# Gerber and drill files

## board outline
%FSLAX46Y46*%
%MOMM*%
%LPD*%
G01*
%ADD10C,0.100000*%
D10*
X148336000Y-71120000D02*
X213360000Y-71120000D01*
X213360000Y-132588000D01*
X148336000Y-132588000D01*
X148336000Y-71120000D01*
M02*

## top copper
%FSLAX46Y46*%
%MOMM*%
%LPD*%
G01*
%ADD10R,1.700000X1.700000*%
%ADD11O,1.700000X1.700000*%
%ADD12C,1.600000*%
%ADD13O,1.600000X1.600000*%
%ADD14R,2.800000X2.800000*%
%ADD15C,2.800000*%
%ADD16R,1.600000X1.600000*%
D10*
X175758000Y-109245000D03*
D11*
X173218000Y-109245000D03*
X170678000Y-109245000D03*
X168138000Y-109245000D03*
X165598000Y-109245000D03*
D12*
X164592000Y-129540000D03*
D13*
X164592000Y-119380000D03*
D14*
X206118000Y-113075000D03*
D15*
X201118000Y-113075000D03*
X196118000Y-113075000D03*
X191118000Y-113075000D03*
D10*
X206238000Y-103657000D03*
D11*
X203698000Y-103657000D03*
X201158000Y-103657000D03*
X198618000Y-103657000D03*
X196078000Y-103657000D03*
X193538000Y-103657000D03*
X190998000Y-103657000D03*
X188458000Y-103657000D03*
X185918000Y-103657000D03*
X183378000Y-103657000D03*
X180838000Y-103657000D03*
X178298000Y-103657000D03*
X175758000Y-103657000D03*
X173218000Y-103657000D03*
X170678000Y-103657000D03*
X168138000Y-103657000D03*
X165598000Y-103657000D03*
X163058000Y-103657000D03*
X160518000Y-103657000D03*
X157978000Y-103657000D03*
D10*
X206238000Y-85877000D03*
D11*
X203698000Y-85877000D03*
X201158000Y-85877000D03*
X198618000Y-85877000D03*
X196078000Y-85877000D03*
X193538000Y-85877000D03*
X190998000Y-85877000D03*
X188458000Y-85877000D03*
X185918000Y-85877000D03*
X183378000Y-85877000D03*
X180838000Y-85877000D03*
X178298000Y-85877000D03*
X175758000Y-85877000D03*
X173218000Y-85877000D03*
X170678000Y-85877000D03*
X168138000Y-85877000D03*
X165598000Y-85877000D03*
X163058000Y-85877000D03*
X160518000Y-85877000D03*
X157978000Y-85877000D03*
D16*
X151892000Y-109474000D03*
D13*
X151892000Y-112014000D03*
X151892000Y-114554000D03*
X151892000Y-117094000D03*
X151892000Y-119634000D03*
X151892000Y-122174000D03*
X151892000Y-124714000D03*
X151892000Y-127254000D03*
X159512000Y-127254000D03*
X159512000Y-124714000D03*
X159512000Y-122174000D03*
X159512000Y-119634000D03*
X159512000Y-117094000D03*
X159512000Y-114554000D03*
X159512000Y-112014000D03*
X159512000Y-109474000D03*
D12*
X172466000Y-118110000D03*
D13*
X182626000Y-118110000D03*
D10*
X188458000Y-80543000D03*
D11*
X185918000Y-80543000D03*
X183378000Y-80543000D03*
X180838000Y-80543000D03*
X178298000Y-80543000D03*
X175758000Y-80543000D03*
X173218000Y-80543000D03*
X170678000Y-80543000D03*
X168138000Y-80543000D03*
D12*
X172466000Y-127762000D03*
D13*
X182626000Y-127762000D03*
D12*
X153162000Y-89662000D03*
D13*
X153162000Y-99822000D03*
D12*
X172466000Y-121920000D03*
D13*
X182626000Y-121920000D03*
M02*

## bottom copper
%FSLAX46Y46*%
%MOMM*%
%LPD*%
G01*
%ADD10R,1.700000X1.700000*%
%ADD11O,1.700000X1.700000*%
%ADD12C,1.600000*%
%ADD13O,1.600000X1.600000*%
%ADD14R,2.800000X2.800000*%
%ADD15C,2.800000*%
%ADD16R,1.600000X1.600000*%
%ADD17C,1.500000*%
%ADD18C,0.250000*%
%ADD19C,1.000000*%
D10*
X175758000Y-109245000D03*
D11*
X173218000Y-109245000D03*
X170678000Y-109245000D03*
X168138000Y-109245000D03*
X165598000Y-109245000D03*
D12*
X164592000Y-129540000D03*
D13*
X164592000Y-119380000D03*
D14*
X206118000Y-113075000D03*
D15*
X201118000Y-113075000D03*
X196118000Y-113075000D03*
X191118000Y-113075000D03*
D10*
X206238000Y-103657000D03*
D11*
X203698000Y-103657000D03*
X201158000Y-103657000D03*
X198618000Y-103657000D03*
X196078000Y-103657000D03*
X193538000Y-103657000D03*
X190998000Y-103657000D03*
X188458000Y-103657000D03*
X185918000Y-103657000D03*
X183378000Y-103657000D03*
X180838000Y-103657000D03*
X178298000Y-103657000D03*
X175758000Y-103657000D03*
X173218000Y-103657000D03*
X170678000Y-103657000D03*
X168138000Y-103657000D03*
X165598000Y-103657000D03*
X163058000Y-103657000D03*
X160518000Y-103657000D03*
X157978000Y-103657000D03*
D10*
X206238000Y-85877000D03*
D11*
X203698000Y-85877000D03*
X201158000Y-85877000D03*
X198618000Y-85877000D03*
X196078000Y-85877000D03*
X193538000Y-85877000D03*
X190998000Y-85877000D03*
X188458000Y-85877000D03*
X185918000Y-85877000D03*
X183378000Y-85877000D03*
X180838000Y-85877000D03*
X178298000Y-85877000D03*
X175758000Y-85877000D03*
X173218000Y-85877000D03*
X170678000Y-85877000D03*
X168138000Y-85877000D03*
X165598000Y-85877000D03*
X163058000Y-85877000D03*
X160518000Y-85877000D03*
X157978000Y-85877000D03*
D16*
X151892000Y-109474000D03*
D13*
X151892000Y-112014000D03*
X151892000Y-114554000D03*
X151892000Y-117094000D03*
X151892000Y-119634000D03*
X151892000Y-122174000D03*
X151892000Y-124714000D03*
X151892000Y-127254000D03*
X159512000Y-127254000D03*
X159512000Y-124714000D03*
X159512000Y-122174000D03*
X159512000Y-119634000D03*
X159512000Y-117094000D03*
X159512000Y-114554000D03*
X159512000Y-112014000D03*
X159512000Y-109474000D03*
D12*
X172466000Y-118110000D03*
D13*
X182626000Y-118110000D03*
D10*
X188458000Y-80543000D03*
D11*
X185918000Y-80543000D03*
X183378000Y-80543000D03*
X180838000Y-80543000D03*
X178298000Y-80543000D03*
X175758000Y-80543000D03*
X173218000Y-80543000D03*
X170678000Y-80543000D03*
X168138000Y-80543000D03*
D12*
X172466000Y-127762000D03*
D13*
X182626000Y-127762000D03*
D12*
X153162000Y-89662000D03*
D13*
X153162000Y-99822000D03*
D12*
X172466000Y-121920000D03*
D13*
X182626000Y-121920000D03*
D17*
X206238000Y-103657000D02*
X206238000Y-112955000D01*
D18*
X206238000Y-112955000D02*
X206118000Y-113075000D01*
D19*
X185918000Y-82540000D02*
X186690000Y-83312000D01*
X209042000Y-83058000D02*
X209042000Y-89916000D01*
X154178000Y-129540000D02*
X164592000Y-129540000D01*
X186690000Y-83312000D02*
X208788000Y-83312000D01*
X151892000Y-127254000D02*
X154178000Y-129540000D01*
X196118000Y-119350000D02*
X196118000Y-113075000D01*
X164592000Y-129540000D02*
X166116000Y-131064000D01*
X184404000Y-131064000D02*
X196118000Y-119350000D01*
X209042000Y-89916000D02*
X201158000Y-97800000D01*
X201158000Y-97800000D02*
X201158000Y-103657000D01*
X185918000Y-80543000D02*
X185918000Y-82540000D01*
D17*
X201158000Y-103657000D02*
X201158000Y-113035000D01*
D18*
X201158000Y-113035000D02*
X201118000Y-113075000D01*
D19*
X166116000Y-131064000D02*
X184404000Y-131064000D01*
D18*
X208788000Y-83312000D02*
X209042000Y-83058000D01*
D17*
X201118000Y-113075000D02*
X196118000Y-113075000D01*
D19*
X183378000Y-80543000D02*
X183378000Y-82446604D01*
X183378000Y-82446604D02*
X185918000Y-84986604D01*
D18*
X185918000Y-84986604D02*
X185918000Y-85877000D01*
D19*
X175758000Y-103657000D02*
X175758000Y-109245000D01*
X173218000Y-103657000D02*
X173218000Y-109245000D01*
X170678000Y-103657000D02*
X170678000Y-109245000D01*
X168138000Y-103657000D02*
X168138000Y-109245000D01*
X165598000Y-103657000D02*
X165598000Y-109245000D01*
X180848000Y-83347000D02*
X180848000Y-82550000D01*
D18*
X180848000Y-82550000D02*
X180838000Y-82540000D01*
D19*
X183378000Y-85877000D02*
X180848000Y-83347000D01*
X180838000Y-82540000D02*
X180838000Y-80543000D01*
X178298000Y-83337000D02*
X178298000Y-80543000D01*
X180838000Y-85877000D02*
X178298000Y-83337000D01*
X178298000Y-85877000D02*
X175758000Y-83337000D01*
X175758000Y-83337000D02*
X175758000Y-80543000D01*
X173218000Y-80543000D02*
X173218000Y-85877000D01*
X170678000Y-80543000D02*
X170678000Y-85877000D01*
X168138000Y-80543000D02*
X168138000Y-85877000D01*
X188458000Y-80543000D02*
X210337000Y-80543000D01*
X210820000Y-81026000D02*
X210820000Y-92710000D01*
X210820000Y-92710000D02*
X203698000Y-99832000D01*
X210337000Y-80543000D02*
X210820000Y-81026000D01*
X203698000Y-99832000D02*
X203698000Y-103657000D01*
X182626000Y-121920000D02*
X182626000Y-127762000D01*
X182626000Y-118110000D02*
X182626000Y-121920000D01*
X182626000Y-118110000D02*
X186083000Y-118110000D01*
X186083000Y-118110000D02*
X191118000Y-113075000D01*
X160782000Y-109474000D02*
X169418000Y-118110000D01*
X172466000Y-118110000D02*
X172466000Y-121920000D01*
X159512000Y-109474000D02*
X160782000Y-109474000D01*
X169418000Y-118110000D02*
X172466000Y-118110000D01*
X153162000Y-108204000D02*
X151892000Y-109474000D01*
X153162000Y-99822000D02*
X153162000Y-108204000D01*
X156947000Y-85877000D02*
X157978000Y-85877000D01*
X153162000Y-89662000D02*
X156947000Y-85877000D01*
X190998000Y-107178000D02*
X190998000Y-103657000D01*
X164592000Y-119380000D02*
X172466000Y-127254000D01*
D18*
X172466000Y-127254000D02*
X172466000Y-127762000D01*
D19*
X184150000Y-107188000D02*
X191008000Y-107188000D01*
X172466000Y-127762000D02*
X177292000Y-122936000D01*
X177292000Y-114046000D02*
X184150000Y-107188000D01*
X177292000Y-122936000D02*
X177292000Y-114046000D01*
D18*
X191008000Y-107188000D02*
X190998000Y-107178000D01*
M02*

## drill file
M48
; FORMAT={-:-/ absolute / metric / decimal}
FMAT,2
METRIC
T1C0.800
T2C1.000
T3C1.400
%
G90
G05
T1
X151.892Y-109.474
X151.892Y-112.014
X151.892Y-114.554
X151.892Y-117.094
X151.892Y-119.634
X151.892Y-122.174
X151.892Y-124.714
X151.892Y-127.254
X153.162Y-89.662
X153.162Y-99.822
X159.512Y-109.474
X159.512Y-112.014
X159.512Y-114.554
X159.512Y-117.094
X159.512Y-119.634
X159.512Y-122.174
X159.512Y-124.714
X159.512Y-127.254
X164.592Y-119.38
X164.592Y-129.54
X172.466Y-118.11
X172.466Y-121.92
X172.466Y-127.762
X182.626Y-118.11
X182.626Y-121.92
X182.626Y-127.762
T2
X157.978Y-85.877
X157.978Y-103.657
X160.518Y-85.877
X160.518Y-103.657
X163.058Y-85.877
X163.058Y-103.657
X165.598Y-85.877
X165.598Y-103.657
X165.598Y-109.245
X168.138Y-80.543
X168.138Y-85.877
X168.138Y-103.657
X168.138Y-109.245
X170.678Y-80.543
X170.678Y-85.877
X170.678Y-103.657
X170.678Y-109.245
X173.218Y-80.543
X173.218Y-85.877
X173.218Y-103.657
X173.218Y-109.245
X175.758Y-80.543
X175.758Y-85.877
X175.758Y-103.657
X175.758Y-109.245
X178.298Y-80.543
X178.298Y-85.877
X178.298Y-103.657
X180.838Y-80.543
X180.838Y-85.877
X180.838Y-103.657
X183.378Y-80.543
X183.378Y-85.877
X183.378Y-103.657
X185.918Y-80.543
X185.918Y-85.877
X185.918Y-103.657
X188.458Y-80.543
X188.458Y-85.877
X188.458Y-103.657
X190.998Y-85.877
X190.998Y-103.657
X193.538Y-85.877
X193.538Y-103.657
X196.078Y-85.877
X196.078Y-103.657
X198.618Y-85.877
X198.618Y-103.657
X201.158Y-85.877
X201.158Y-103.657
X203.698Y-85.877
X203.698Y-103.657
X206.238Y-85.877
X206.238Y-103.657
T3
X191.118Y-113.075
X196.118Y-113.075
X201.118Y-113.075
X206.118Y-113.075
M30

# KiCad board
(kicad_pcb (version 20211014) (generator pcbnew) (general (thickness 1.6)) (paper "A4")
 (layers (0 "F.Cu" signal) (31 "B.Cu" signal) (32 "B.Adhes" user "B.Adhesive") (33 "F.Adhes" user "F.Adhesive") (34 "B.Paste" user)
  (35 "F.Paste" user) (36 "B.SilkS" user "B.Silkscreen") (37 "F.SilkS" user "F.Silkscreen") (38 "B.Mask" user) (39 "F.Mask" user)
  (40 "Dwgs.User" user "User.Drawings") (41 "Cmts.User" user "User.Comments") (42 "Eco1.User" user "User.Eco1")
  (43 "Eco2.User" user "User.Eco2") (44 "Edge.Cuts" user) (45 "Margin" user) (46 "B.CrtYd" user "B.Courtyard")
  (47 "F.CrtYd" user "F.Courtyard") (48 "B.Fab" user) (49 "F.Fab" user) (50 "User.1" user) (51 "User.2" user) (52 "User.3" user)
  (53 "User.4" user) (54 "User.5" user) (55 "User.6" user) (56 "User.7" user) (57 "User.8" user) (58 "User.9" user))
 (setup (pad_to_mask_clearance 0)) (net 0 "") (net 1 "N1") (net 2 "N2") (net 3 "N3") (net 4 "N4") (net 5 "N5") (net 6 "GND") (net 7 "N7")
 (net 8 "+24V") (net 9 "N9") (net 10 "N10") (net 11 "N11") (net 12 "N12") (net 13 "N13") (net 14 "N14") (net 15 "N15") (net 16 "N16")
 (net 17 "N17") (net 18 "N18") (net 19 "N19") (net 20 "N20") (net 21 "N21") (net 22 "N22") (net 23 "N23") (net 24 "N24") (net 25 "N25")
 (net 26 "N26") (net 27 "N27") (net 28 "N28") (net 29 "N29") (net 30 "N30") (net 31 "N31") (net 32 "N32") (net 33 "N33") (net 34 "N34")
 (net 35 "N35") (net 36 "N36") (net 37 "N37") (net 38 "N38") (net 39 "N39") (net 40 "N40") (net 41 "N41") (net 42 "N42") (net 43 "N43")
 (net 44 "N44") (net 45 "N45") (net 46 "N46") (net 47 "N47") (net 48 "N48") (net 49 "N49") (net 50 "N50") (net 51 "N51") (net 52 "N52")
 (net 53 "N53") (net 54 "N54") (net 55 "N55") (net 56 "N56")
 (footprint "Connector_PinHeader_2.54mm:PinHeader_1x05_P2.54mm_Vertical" (layer "F.Cu") (at 175.758 109.245 -90)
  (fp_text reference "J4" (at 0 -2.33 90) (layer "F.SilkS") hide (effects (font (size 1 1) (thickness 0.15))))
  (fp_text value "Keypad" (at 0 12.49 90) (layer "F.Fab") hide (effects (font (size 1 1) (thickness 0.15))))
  (pad "1" thru_hole rect (at 0 0 270) (size 1.7 1.7) (drill 1) (layers *.Cu *.Mask) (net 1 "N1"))
  (pad "2" thru_hole oval (at 0 2.54 270) (size 1.7 1.7) (drill 1) (layers *.Cu *.Mask) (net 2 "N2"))
  (pad "3" thru_hole oval (at 0 5.08 270) (size 1.7 1.7) (drill 1) (layers *.Cu *.Mask) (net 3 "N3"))
  (pad "4" thru_hole oval (at 0 7.62 270) (size 1.7 1.7) (drill 1) (layers *.Cu *.Mask) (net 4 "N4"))
  (pad "5" thru_hole oval (at 0 10.16 270) (size 1.7 1.7) (drill 1) (layers *.Cu *.Mask) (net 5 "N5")))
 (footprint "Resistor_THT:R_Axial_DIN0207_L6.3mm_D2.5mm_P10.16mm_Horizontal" (layer "F.Cu") (at 164.592 129.54 90)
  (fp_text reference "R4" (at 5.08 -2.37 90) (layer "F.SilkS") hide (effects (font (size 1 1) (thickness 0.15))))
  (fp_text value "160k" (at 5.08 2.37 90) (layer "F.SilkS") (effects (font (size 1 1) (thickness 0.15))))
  (pad "1" thru_hole circle (at 0 0 90) (size 1.6 1.6) (drill 0.8) (layers *.Cu *.Mask) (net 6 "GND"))
  (pad "2" thru_hole oval (at 10.16 0 90) (size 1.6 1.6) (drill 0.8) (layers *.Cu *.Mask) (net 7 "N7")))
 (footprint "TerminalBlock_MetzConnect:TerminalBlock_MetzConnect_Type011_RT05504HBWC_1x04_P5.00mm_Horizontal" (layer "F.Cu")
  (at 206.118 113.075 180)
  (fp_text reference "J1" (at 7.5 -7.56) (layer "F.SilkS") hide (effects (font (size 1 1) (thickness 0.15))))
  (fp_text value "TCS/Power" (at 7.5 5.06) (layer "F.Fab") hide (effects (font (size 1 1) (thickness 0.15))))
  (pad "1" thru_hole rect (at 0 0 180) (size 2.8 2.8) (drill 1.4) (layers *.Cu *.Mask) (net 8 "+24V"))
  (pad "2" thru_hole circle (at 5 0 180) (size 2.8 2.8) (drill 1.4) (layers *.Cu *.Mask) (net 6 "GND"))
  (pad "3" thru_hole circle (at 10 0 180) (size 2.8 2.8) (drill 1.4) (layers *.Cu *.Mask) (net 6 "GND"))
  (pad "4" thru_hole circle (at 15 0 180) (size 2.8 2.8) (drill 1.4) (layers *.Cu *.Mask) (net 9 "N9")))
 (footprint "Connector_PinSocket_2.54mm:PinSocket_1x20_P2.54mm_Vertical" (layer "F.Cu") (at 206.238 103.657 -90)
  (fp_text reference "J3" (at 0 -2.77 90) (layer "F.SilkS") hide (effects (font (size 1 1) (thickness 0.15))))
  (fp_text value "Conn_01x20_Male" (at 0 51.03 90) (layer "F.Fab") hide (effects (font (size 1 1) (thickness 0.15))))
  (pad "1" thru_hole rect (at 0 0 270) (size 1.7 1.7) (drill 1) (layers *.Cu *.Mask) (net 8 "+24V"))
  (pad "2" thru_hole oval (at 0 2.54 270) (size 1.7 1.7) (drill 1) (layers *.Cu *.Mask) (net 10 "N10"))
  (pad "3" thru_hole oval (at 0 5.08 270) (size 1.7 1.7) (drill 1) (layers *.Cu *.Mask) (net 6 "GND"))
  (pad "4" thru_hole oval (at 0 7.62 270) (size 1.7 1.7) (drill 1) (layers *.Cu *.Mask) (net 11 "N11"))
  (pad "5" thru_hole oval (at 0 10.16 270) (size 1.7 1.7) (drill 1) (layers *.Cu *.Mask) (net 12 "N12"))
  (pad "6" thru_hole oval (at 0 12.7 270) (size 1.7 1.7) (drill 1) (layers *.Cu *.Mask) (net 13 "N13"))
  (pad "7" thru_hole oval (at 0 15.24 270) (size 1.7 1.7) (drill 1) (layers *.Cu *.Mask) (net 7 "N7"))
  (pad "8" thru_hole oval (at 0 17.78 270) (size 1.7 1.7) (drill 1) (layers *.Cu *.Mask) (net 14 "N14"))
  (pad "9" thru_hole oval (at 0 20.32 270) (size 1.7 1.7) (drill 1) (layers *.Cu *.Mask) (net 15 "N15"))
  (pad "10" thru_hole oval (at 0 22.86 270) (size 1.7 1.7) (drill 1) (layers *.Cu *.Mask) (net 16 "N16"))
  (pad "11" thru_hole oval (at 0 25.4 270) (size 1.7 1.7) (drill 1) (layers *.Cu *.Mask) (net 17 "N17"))
  (pad "12" thru_hole oval (at 0 27.94 270) (size 1.7 1.7) (drill 1) (layers *.Cu *.Mask) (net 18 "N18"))
  (pad "13" thru_hole oval (at 0 30.48 270) (size 1.7 1.7) (drill 1) (layers *.Cu *.Mask) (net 1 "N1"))
  (pad "14" thru_hole oval (at 0 33.02 270) (size 1.7 1.7) (drill 1) (layers *.Cu *.Mask) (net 2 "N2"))
  (pad "15" thru_hole oval (at 0 35.56 270) (size 1.7 1.7) (drill 1) (layers *.Cu *.Mask) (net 3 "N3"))
  (pad "16" thru_hole oval (at 0 38.1 270) (size 1.7 1.7) (drill 1) (layers *.Cu *.Mask) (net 4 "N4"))
  (pad "17" thru_hole oval (at 0 40.64 270) (size 1.7 1.7) (drill 1) (layers *.Cu *.Mask) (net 5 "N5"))
  (pad "18" thru_hole oval (at 0 43.18 270) (size 1.7 1.7) (drill 1) (layers *.Cu *.Mask) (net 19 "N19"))
  (pad "19" thru_hole oval (at 0 45.72 270) (size 1.7 1.7) (drill 1) (layers *.Cu *.Mask) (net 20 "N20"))
  (pad "20" thru_hole oval (at 0 48.26 270) (size 1.7 1.7) (drill 1) (layers *.Cu *.Mask) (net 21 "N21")))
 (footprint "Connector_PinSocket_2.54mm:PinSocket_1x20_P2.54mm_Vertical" (layer "F.Cu") (at 206.238 85.877 -90)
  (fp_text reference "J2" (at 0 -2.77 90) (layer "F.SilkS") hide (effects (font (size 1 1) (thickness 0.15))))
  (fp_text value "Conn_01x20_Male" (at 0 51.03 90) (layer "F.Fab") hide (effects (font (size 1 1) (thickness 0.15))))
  (pad "1" thru_hole rect (at 0 0 270) (size 1.7 1.7) (drill 1) (layers *.Cu *.Mask) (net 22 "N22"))
  (pad "2" thru_hole oval (at 0 2.54 270) (size 1.7 1.7) (drill 1) (layers *.Cu *.Mask) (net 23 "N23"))
  (pad "3" thru_hole oval (at 0 5.08 270) (size 1.7 1.7) (drill 1) (layers *.Cu *.Mask) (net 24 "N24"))
  (pad "4" thru_hole oval (at 0 7.62 270) (size 1.7 1.7) (drill 1) (layers *.Cu *.Mask) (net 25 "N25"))
  (pad "5" thru_hole oval (at 0 10.16 270) (size 1.7 1.7) (drill 1) (layers *.Cu *.Mask) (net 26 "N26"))
  (pad "6" thru_hole oval (at 0 12.7 270) (size 1.7 1.7) (drill 1) (layers *.Cu *.Mask) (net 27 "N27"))
  (pad "7" thru_hole oval (at 0 15.24 270) (size 1.7 1.7) (drill 1) (layers *.Cu *.Mask) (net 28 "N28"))
  (pad "8" thru_hole oval (at 0 17.78 270) (size 1.7 1.7) (drill 1) (layers *.Cu *.Mask) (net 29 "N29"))
  (pad "9" thru_hole oval (at 0 20.32 270) (size 1.7 1.7) (drill 1) (layers *.Cu *.Mask) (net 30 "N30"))
  (pad "10" thru_hole oval (at 0 22.86 270) (size 1.7 1.7) (drill 1) (layers *.Cu *.Mask) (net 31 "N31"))
  (pad "11" thru_hole oval (at 0 25.4 270) (size 1.7 1.7) (drill 1) (layers *.Cu *.Mask) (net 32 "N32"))
  (pad "12" thru_hole oval (at 0 27.94 270) (size 1.7 1.7) (drill 1) (layers *.Cu *.Mask) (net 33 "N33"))
  (pad "13" thru_hole oval (at 0 30.48 270) (size 1.7 1.7) (drill 1) (layers *.Cu *.Mask) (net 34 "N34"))
  (pad "14" thru_hole oval (at 0 33.02 270) (size 1.7 1.7) (drill 1) (layers *.Cu *.Mask) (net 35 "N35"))
  (pad "15" thru_hole oval (at 0 35.56 270) (size 1.7 1.7) (drill 1) (layers *.Cu *.Mask) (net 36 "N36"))
  (pad "16" thru_hole oval (at 0 38.1 270) (size 1.7 1.7) (drill 1) (layers *.Cu *.Mask) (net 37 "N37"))
  (pad "17" thru_hole oval (at 0 40.64 270) (size 1.7 1.7) (drill 1) (layers *.Cu *.Mask) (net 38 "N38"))
  (pad "18" thru_hole oval (at 0 43.18 270) (size 1.7 1.7) (drill 1) (layers *.Cu *.Mask) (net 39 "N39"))
  (pad "19" thru_hole oval (at 0 45.72 270) (size 1.7 1.7) (drill 1) (layers *.Cu *.Mask) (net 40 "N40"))
  (pad "20" thru_hole oval (at 0 48.26 270) (size 1.7 1.7) (drill 1) (layers *.Cu *.Mask) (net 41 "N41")))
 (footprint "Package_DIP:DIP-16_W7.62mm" (layer "F.Cu") (at 151.892 109.474)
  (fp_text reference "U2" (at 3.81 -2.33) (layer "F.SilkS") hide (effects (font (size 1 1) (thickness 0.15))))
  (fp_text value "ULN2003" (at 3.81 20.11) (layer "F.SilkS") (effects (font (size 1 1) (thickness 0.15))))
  (pad "1" thru_hole rect (at 0 0) (size 1.6 1.6) (drill 0.8) (layers *.Cu *.Mask) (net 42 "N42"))
  (pad "2" thru_hole oval (at 0 2.54) (size 1.6 1.6) (drill 0.8) (layers *.Cu *.Mask) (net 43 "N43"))
  (pad "3" thru_hole oval (at 0 5.08) (size 1.6 1.6) (drill 0.8) (layers *.Cu *.Mask) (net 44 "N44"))
  (pad "4" thru_hole oval (at 0 7.62) (size 1.6 1.6) (drill 0.8) (layers *.Cu *.Mask) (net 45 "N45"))
  (pad "5" thru_hole oval (at 0 10.16) (size 1.6 1.6) (drill 0.8) (layers *.Cu *.Mask) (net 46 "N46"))
  (pad "6" thru_hole oval (at 0 12.7) (size 1.6 1.6) (drill 0.8) (layers *.Cu *.Mask) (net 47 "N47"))
  (pad "7" thru_hole oval (at 0 15.24) (size 1.6 1.6) (drill 0.8) (layers *.Cu *.Mask) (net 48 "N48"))
  (pad "8" thru_hole oval (at 0 17.78) (size 1.6 1.6) (drill 0.8) (layers *.Cu *.Mask) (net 6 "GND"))
  (pad "9" thru_hole oval (at 7.62 17.78) (size 1.6 1.6) (drill 0.8) (layers *.Cu *.Mask) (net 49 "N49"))
  (pad "10" thru_hole oval (at 7.62 15.24) (size 1.6 1.6) (drill 0.8) (layers *.Cu *.Mask) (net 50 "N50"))
  (pad "11" thru_hole oval (at 7.62 12.7) (size 1.6 1.6) (drill 0.8) (layers *.Cu *.Mask) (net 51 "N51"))
  (pad "12" thru_hole oval (at 7.62 10.16) (size 1.6 1.6) (drill 0.8) (layers *.Cu *.Mask) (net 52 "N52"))
  (pad "13" thru_hole oval (at 7.62 7.62) (size 1.6 1.6) (drill 0.8) (layers *.Cu *.Mask) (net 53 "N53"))
  (pad "14" thru_hole oval (at 7.62 5.08) (size 1.6 1.6) (drill 0.8) (layers *.Cu *.Mask) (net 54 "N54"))
  (pad "15" thru_hole oval (at 7.62 2.54) (size 1.6 1.6) (drill 0.8) (layers *.Cu *.Mask) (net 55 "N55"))
  (pad "16" thru_hole oval (at 7.62 0) (size 1.6 1.6) (drill 0.8) (layers *.Cu *.Mask) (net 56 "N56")))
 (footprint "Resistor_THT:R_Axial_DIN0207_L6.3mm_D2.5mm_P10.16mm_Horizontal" (layer "F.Cu") (at 172.466 118.11)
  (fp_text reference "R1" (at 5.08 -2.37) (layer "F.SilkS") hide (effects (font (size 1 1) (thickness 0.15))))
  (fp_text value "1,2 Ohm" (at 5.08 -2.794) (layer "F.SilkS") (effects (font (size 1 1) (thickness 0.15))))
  (pad "1" thru_hole circle (at 0 0) (size 1.6 1.6) (drill 0.8) (layers *.Cu *.Mask) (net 56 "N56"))
  (pad "2" thru_hole oval (at 10.16 0) (size 1.6 1.6) (drill 0.8) (layers *.Cu *.Mask) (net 9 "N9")))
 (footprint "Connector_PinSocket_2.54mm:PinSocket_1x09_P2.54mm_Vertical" (layer "F.Cu") (at 188.458 80.543 -90)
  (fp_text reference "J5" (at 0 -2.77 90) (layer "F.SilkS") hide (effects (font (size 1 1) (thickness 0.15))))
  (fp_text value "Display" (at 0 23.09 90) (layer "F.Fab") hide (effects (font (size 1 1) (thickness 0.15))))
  (pad "1" thru_hole rect (at 0 0 270) (size 1.7 1.7) (drill 1) (layers *.Cu *.Mask) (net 10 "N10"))
  (pad "2" thru_hole oval (at 0 2.54 270) (size 1.7 1.7) (drill 1) (layers *.Cu *.Mask) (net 6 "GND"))
  (pad "3" thru_hole oval (at 0 5.08 270) (size 1.7 1.7) (drill 1) (layers *.Cu *.Mask) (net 30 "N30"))
  (pad "4" thru_hole oval (at 0 7.62 270) (size 1.7 1.7) (drill 1) (layers *.Cu *.Mask) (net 31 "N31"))
  (pad "5" thru_hole oval (at 0 10.16 270) (size 1.7 1.7) (drill 1) (layers *.Cu *.Mask) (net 32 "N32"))
  (pad "6" thru_hole oval (at 0 12.7 270) (size 1.7 1.7) (drill 1) (layers *.Cu *.Mask) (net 33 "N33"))
  (pad "7" thru_hole oval (at 0 15.24 270) (size 1.7 1.7) (drill 1) (layers *.Cu *.Mask) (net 35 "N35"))
  (pad "8" thru_hole oval (at 0 17.78 270) (size 1.7 1.7) (drill 1) (layers *.Cu *.Mask) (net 36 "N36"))
  (pad "9" thru_hole oval (at 0 20.32 270) (size 1.7 1.7) (drill 1) (layers *.Cu *.Mask) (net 37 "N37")))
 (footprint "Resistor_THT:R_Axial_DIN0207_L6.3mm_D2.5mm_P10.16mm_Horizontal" (layer "F.Cu") (at 172.466 127.762)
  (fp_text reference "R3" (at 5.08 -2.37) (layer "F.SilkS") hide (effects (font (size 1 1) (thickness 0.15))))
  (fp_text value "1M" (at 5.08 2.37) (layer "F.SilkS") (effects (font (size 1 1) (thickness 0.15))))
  (pad "1" thru_hole circle (at 0 0) (size 1.6 1.6) (drill 0.8) (layers *.Cu *.Mask) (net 7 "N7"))
  (pad "2" thru_hole oval (at 10.16 0) (size 1.6 1.6) (drill 0.8) (layers *.Cu *.Mask) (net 9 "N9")))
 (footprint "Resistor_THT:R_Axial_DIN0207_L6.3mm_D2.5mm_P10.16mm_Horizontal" (layer "F.Cu") (at 153.162 89.662 -90)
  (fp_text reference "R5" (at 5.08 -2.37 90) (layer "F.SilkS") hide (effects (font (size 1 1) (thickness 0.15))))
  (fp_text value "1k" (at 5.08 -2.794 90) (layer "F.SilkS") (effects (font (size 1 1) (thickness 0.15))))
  (pad "1" thru_hole circle (at 0 0 270) (size 1.6 1.6) (drill 0.8) (layers *.Cu *.Mask) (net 41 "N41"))
  (pad "2" thru_hole oval (at 10.16 0 270) (size 1.6 1.6) (drill 0.8) (layers *.Cu *.Mask) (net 42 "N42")))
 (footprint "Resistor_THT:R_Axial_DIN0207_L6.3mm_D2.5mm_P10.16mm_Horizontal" (layer "F.Cu") (at 172.466 121.92)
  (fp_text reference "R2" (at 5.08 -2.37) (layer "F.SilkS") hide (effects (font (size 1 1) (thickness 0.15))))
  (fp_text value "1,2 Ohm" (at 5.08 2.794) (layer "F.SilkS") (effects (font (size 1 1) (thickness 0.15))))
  (pad "1" thru_hole circle (at 0 0) (size 1.6 1.6) (drill 0.8) (layers *.Cu *.Mask) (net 56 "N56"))
  (pad "2" thru_hole oval (at 10.16 0) (size 1.6 1.6) (drill 0.8) (layers *.Cu *.Mask) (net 9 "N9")))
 (gr_rect (start 148.336 71.12) (end 213.36 132.588) (layer "Edge.Cuts") (width 0.1) (fill none))
 (segment (start 206.238 103.657) (end 206.238 112.955) (width 1.5) (layer "B.Cu") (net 8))
 (segment (start 206.238 112.955) (end 206.118 113.075) (width 0.25) (layer "B.Cu") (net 8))
 (segment (start 185.918 82.54) (end 186.69 83.312) (width 1) (layer "B.Cu") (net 6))
 (segment (start 209.042 83.058) (end 209.042 89.916) (width 1) (layer "B.Cu") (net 6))
 (segment (start 154.178 129.54) (end 164.592 129.54) (width 1) (layer "B.Cu") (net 6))
 (segment (start 186.69 83.312) (end 208.788 83.312) (width 1) (layer "B.Cu") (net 6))
 (segment (start 151.892 127.254) (end 154.178 129.54) (width 1) (layer "B.Cu") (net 6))
 (segment (start 196.118 119.35) (end 196.118 113.075) (width 1) (layer "B.Cu") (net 6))
 (segment (start 164.592 129.54) (end 166.116 131.064) (width 1) (layer "B.Cu") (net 6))
 (segment (start 184.404 131.064) (end 196.118 119.35) (width 1) (layer "B.Cu") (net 6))
 (segment (start 209.042 89.916) (end 201.158 97.8) (width 1) (layer "B.Cu") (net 6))
 (segment (start 201.158 97.8) (end 201.158 103.657) (width 1) (layer "B.Cu") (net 6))
 (segment (start 185.918 80.543) (end 185.918 82.54) (width 1) (layer "B.Cu") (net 6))
 (segment (start 201.158 103.657) (end 201.158 113.035) (width 1.5) (layer "B.Cu") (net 6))
 (segment (start 201.158 113.035) (end 201.118 113.075) (width 0.25) (layer "B.Cu") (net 6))
 (segment (start 166.116 131.064) (end 184.404 131.064) (width 1) (layer "B.Cu") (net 6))
 (segment (start 208.788 83.312) (end 209.042 83.058) (width 0.25) (layer "B.Cu") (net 6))
 (segment (start 201.118 113.075) (end 196.118 113.075) (width 1.5) (layer "B.Cu") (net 6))
 (segment (start 183.378 80.543) (end 183.378 82.446604) (width 1) (layer "B.Cu") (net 30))
 (segment (start 183.378 82.446604) (end 185.918 84.986604) (width 1) (layer "B.Cu") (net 30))
 (segment (start 185.918 84.986604) (end 185.918 85.877) (width 0.25) (layer "B.Cu") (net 30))
 (segment (start 175.758 103.657) (end 175.758 109.245) (width 1) (layer "B.Cu") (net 1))
 (segment (start 173.218 103.657) (end 173.218 109.245) (width 1) (layer "B.Cu") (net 2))
 (segment (start 170.678 103.657) (end 170.678 109.245) (width 1) (layer "B.Cu") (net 3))
 (segment (start 168.138 103.657) (end 168.138 109.245) (width 1) (layer "B.Cu") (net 4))
 (segment (start 165.598 103.657) (end 165.598 109.245) (width 1) (layer "B.Cu") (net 5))
 (segment (start 180.848 83.347) (end 180.848 82.55) (width 1) (layer "B.Cu") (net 31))
 (segment (start 180.848 82.55) (end 180.838 82.54) (width 0.25) (layer "B.Cu") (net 31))
 (segment (start 183.378 85.877) (end 180.848 83.347) (width 1) (layer "B.Cu") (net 31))
 (segment (start 180.838 82.54) (end 180.838 80.543) (width 1) (layer "B.Cu") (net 31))
 (segment (start 178.298 83.337) (end 178.298 80.543) (width 1) (layer "B.Cu") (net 32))
 (segment (start 180.838 85.877) (end 178.298 83.337) (width 1) (layer "B.Cu") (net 32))
 (segment (start 178.298 85.877) (end 175.758 83.337) (width 1) (layer "B.Cu") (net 33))
 (segment (start 175.758 83.337) (end 175.758 80.543) (width 1) (layer "B.Cu") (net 33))
 (segment (start 173.218 80.543) (end 173.218 85.877) (width 1) (layer "B.Cu") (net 35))
 (segment (start 170.678 80.543) (end 170.678 85.877) (width 1) (layer "B.Cu") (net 36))
 (segment (start 168.138 80.543) (end 168.138 85.877) (width 1) (layer "B.Cu") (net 37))
 (segment (start 188.458 80.543) (end 210.337 80.543) (width 1) (layer "B.Cu") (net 10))
 (segment (start 210.82 81.026) (end 210.82 92.71) (width 1) (layer "B.Cu") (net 10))
 (segment (start 210.82 92.71) (end 203.698 99.832) (width 1) (layer "B.Cu") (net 10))
 (segment (start 210.337 80.543) (end 210.82 81.026) (width 1) (layer "B.Cu") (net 10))
 (segment (start 203.698 99.832) (end 203.698 103.657) (width 1) (layer "B.Cu") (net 10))
 (segment (start 182.626 121.92) (end 182.626 127.762) (width 1) (layer "B.Cu") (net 9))
 (segment (start 182.626 118.11) (end 182.626 121.92) (width 1) (layer "B.Cu") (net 9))
 (segment (start 182.626 118.11) (end 186.083 118.11) (width 1) (layer "B.Cu") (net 9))
 (segment (start 186.083 118.11) (end 191.118 113.075) (width 1) (layer "B.Cu") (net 9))
 (segment (start 160.782 109.474) (end 169.418 118.11) (width 1) (layer "B.Cu") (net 56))
 (segment (start 172.466 118.11) (end 172.466 121.92) (width 1) (layer "B.Cu") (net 56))
 (segment (start 159.512 109.474) (end 160.782 109.474) (width 1) (layer "B.Cu") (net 56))
 (segment (start 169.418 118.11) (end 172.466 118.11) (width 1) (layer "B.Cu") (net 56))
 (segment (start 153.162 108.204) (end 151.892 109.474) (width 1) (layer "B.Cu") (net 42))
 (segment (start 153.162 99.822) (end 153.162 108.204) (width 1) (layer "B.Cu") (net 42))
 (segment (start 156.947 85.877) (end 157.978 85.877) (width 1) (layer "B.Cu") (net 41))
 (segment (start 153.162 89.662) (end 156.947 85.877) (width 1) (layer "B.Cu") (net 41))
 (segment (start 190.998 107.178) (end 190.998 103.657) (width 1) (layer "B.Cu") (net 7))
 (segment (start 164.592 119.38) (end 172.466 127.254) (width 1) (layer "B.Cu") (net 7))
 (segment (start 172.466 127.254) (end 172.466 127.762) (width 0.25) (layer "B.Cu") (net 7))
 (segment (start 184.15 107.188) (end 191.008 107.188) (width 1) (layer "B.Cu") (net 7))
 (segment (start 172.466 127.762) (end 177.292 122.936) (width 1) (layer "B.Cu") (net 7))
 (segment (start 177.292 114.046) (end 184.15 107.188) (width 1) (layer "B.Cu") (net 7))
 (segment (start 177.292 122.936) (end 177.292 114.046) (width 1) (layer "B.Cu") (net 7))
 (segment (start 191.008 107.188) (end 190.998 107.178) (width 0.25) (layer "B.Cu") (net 7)))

